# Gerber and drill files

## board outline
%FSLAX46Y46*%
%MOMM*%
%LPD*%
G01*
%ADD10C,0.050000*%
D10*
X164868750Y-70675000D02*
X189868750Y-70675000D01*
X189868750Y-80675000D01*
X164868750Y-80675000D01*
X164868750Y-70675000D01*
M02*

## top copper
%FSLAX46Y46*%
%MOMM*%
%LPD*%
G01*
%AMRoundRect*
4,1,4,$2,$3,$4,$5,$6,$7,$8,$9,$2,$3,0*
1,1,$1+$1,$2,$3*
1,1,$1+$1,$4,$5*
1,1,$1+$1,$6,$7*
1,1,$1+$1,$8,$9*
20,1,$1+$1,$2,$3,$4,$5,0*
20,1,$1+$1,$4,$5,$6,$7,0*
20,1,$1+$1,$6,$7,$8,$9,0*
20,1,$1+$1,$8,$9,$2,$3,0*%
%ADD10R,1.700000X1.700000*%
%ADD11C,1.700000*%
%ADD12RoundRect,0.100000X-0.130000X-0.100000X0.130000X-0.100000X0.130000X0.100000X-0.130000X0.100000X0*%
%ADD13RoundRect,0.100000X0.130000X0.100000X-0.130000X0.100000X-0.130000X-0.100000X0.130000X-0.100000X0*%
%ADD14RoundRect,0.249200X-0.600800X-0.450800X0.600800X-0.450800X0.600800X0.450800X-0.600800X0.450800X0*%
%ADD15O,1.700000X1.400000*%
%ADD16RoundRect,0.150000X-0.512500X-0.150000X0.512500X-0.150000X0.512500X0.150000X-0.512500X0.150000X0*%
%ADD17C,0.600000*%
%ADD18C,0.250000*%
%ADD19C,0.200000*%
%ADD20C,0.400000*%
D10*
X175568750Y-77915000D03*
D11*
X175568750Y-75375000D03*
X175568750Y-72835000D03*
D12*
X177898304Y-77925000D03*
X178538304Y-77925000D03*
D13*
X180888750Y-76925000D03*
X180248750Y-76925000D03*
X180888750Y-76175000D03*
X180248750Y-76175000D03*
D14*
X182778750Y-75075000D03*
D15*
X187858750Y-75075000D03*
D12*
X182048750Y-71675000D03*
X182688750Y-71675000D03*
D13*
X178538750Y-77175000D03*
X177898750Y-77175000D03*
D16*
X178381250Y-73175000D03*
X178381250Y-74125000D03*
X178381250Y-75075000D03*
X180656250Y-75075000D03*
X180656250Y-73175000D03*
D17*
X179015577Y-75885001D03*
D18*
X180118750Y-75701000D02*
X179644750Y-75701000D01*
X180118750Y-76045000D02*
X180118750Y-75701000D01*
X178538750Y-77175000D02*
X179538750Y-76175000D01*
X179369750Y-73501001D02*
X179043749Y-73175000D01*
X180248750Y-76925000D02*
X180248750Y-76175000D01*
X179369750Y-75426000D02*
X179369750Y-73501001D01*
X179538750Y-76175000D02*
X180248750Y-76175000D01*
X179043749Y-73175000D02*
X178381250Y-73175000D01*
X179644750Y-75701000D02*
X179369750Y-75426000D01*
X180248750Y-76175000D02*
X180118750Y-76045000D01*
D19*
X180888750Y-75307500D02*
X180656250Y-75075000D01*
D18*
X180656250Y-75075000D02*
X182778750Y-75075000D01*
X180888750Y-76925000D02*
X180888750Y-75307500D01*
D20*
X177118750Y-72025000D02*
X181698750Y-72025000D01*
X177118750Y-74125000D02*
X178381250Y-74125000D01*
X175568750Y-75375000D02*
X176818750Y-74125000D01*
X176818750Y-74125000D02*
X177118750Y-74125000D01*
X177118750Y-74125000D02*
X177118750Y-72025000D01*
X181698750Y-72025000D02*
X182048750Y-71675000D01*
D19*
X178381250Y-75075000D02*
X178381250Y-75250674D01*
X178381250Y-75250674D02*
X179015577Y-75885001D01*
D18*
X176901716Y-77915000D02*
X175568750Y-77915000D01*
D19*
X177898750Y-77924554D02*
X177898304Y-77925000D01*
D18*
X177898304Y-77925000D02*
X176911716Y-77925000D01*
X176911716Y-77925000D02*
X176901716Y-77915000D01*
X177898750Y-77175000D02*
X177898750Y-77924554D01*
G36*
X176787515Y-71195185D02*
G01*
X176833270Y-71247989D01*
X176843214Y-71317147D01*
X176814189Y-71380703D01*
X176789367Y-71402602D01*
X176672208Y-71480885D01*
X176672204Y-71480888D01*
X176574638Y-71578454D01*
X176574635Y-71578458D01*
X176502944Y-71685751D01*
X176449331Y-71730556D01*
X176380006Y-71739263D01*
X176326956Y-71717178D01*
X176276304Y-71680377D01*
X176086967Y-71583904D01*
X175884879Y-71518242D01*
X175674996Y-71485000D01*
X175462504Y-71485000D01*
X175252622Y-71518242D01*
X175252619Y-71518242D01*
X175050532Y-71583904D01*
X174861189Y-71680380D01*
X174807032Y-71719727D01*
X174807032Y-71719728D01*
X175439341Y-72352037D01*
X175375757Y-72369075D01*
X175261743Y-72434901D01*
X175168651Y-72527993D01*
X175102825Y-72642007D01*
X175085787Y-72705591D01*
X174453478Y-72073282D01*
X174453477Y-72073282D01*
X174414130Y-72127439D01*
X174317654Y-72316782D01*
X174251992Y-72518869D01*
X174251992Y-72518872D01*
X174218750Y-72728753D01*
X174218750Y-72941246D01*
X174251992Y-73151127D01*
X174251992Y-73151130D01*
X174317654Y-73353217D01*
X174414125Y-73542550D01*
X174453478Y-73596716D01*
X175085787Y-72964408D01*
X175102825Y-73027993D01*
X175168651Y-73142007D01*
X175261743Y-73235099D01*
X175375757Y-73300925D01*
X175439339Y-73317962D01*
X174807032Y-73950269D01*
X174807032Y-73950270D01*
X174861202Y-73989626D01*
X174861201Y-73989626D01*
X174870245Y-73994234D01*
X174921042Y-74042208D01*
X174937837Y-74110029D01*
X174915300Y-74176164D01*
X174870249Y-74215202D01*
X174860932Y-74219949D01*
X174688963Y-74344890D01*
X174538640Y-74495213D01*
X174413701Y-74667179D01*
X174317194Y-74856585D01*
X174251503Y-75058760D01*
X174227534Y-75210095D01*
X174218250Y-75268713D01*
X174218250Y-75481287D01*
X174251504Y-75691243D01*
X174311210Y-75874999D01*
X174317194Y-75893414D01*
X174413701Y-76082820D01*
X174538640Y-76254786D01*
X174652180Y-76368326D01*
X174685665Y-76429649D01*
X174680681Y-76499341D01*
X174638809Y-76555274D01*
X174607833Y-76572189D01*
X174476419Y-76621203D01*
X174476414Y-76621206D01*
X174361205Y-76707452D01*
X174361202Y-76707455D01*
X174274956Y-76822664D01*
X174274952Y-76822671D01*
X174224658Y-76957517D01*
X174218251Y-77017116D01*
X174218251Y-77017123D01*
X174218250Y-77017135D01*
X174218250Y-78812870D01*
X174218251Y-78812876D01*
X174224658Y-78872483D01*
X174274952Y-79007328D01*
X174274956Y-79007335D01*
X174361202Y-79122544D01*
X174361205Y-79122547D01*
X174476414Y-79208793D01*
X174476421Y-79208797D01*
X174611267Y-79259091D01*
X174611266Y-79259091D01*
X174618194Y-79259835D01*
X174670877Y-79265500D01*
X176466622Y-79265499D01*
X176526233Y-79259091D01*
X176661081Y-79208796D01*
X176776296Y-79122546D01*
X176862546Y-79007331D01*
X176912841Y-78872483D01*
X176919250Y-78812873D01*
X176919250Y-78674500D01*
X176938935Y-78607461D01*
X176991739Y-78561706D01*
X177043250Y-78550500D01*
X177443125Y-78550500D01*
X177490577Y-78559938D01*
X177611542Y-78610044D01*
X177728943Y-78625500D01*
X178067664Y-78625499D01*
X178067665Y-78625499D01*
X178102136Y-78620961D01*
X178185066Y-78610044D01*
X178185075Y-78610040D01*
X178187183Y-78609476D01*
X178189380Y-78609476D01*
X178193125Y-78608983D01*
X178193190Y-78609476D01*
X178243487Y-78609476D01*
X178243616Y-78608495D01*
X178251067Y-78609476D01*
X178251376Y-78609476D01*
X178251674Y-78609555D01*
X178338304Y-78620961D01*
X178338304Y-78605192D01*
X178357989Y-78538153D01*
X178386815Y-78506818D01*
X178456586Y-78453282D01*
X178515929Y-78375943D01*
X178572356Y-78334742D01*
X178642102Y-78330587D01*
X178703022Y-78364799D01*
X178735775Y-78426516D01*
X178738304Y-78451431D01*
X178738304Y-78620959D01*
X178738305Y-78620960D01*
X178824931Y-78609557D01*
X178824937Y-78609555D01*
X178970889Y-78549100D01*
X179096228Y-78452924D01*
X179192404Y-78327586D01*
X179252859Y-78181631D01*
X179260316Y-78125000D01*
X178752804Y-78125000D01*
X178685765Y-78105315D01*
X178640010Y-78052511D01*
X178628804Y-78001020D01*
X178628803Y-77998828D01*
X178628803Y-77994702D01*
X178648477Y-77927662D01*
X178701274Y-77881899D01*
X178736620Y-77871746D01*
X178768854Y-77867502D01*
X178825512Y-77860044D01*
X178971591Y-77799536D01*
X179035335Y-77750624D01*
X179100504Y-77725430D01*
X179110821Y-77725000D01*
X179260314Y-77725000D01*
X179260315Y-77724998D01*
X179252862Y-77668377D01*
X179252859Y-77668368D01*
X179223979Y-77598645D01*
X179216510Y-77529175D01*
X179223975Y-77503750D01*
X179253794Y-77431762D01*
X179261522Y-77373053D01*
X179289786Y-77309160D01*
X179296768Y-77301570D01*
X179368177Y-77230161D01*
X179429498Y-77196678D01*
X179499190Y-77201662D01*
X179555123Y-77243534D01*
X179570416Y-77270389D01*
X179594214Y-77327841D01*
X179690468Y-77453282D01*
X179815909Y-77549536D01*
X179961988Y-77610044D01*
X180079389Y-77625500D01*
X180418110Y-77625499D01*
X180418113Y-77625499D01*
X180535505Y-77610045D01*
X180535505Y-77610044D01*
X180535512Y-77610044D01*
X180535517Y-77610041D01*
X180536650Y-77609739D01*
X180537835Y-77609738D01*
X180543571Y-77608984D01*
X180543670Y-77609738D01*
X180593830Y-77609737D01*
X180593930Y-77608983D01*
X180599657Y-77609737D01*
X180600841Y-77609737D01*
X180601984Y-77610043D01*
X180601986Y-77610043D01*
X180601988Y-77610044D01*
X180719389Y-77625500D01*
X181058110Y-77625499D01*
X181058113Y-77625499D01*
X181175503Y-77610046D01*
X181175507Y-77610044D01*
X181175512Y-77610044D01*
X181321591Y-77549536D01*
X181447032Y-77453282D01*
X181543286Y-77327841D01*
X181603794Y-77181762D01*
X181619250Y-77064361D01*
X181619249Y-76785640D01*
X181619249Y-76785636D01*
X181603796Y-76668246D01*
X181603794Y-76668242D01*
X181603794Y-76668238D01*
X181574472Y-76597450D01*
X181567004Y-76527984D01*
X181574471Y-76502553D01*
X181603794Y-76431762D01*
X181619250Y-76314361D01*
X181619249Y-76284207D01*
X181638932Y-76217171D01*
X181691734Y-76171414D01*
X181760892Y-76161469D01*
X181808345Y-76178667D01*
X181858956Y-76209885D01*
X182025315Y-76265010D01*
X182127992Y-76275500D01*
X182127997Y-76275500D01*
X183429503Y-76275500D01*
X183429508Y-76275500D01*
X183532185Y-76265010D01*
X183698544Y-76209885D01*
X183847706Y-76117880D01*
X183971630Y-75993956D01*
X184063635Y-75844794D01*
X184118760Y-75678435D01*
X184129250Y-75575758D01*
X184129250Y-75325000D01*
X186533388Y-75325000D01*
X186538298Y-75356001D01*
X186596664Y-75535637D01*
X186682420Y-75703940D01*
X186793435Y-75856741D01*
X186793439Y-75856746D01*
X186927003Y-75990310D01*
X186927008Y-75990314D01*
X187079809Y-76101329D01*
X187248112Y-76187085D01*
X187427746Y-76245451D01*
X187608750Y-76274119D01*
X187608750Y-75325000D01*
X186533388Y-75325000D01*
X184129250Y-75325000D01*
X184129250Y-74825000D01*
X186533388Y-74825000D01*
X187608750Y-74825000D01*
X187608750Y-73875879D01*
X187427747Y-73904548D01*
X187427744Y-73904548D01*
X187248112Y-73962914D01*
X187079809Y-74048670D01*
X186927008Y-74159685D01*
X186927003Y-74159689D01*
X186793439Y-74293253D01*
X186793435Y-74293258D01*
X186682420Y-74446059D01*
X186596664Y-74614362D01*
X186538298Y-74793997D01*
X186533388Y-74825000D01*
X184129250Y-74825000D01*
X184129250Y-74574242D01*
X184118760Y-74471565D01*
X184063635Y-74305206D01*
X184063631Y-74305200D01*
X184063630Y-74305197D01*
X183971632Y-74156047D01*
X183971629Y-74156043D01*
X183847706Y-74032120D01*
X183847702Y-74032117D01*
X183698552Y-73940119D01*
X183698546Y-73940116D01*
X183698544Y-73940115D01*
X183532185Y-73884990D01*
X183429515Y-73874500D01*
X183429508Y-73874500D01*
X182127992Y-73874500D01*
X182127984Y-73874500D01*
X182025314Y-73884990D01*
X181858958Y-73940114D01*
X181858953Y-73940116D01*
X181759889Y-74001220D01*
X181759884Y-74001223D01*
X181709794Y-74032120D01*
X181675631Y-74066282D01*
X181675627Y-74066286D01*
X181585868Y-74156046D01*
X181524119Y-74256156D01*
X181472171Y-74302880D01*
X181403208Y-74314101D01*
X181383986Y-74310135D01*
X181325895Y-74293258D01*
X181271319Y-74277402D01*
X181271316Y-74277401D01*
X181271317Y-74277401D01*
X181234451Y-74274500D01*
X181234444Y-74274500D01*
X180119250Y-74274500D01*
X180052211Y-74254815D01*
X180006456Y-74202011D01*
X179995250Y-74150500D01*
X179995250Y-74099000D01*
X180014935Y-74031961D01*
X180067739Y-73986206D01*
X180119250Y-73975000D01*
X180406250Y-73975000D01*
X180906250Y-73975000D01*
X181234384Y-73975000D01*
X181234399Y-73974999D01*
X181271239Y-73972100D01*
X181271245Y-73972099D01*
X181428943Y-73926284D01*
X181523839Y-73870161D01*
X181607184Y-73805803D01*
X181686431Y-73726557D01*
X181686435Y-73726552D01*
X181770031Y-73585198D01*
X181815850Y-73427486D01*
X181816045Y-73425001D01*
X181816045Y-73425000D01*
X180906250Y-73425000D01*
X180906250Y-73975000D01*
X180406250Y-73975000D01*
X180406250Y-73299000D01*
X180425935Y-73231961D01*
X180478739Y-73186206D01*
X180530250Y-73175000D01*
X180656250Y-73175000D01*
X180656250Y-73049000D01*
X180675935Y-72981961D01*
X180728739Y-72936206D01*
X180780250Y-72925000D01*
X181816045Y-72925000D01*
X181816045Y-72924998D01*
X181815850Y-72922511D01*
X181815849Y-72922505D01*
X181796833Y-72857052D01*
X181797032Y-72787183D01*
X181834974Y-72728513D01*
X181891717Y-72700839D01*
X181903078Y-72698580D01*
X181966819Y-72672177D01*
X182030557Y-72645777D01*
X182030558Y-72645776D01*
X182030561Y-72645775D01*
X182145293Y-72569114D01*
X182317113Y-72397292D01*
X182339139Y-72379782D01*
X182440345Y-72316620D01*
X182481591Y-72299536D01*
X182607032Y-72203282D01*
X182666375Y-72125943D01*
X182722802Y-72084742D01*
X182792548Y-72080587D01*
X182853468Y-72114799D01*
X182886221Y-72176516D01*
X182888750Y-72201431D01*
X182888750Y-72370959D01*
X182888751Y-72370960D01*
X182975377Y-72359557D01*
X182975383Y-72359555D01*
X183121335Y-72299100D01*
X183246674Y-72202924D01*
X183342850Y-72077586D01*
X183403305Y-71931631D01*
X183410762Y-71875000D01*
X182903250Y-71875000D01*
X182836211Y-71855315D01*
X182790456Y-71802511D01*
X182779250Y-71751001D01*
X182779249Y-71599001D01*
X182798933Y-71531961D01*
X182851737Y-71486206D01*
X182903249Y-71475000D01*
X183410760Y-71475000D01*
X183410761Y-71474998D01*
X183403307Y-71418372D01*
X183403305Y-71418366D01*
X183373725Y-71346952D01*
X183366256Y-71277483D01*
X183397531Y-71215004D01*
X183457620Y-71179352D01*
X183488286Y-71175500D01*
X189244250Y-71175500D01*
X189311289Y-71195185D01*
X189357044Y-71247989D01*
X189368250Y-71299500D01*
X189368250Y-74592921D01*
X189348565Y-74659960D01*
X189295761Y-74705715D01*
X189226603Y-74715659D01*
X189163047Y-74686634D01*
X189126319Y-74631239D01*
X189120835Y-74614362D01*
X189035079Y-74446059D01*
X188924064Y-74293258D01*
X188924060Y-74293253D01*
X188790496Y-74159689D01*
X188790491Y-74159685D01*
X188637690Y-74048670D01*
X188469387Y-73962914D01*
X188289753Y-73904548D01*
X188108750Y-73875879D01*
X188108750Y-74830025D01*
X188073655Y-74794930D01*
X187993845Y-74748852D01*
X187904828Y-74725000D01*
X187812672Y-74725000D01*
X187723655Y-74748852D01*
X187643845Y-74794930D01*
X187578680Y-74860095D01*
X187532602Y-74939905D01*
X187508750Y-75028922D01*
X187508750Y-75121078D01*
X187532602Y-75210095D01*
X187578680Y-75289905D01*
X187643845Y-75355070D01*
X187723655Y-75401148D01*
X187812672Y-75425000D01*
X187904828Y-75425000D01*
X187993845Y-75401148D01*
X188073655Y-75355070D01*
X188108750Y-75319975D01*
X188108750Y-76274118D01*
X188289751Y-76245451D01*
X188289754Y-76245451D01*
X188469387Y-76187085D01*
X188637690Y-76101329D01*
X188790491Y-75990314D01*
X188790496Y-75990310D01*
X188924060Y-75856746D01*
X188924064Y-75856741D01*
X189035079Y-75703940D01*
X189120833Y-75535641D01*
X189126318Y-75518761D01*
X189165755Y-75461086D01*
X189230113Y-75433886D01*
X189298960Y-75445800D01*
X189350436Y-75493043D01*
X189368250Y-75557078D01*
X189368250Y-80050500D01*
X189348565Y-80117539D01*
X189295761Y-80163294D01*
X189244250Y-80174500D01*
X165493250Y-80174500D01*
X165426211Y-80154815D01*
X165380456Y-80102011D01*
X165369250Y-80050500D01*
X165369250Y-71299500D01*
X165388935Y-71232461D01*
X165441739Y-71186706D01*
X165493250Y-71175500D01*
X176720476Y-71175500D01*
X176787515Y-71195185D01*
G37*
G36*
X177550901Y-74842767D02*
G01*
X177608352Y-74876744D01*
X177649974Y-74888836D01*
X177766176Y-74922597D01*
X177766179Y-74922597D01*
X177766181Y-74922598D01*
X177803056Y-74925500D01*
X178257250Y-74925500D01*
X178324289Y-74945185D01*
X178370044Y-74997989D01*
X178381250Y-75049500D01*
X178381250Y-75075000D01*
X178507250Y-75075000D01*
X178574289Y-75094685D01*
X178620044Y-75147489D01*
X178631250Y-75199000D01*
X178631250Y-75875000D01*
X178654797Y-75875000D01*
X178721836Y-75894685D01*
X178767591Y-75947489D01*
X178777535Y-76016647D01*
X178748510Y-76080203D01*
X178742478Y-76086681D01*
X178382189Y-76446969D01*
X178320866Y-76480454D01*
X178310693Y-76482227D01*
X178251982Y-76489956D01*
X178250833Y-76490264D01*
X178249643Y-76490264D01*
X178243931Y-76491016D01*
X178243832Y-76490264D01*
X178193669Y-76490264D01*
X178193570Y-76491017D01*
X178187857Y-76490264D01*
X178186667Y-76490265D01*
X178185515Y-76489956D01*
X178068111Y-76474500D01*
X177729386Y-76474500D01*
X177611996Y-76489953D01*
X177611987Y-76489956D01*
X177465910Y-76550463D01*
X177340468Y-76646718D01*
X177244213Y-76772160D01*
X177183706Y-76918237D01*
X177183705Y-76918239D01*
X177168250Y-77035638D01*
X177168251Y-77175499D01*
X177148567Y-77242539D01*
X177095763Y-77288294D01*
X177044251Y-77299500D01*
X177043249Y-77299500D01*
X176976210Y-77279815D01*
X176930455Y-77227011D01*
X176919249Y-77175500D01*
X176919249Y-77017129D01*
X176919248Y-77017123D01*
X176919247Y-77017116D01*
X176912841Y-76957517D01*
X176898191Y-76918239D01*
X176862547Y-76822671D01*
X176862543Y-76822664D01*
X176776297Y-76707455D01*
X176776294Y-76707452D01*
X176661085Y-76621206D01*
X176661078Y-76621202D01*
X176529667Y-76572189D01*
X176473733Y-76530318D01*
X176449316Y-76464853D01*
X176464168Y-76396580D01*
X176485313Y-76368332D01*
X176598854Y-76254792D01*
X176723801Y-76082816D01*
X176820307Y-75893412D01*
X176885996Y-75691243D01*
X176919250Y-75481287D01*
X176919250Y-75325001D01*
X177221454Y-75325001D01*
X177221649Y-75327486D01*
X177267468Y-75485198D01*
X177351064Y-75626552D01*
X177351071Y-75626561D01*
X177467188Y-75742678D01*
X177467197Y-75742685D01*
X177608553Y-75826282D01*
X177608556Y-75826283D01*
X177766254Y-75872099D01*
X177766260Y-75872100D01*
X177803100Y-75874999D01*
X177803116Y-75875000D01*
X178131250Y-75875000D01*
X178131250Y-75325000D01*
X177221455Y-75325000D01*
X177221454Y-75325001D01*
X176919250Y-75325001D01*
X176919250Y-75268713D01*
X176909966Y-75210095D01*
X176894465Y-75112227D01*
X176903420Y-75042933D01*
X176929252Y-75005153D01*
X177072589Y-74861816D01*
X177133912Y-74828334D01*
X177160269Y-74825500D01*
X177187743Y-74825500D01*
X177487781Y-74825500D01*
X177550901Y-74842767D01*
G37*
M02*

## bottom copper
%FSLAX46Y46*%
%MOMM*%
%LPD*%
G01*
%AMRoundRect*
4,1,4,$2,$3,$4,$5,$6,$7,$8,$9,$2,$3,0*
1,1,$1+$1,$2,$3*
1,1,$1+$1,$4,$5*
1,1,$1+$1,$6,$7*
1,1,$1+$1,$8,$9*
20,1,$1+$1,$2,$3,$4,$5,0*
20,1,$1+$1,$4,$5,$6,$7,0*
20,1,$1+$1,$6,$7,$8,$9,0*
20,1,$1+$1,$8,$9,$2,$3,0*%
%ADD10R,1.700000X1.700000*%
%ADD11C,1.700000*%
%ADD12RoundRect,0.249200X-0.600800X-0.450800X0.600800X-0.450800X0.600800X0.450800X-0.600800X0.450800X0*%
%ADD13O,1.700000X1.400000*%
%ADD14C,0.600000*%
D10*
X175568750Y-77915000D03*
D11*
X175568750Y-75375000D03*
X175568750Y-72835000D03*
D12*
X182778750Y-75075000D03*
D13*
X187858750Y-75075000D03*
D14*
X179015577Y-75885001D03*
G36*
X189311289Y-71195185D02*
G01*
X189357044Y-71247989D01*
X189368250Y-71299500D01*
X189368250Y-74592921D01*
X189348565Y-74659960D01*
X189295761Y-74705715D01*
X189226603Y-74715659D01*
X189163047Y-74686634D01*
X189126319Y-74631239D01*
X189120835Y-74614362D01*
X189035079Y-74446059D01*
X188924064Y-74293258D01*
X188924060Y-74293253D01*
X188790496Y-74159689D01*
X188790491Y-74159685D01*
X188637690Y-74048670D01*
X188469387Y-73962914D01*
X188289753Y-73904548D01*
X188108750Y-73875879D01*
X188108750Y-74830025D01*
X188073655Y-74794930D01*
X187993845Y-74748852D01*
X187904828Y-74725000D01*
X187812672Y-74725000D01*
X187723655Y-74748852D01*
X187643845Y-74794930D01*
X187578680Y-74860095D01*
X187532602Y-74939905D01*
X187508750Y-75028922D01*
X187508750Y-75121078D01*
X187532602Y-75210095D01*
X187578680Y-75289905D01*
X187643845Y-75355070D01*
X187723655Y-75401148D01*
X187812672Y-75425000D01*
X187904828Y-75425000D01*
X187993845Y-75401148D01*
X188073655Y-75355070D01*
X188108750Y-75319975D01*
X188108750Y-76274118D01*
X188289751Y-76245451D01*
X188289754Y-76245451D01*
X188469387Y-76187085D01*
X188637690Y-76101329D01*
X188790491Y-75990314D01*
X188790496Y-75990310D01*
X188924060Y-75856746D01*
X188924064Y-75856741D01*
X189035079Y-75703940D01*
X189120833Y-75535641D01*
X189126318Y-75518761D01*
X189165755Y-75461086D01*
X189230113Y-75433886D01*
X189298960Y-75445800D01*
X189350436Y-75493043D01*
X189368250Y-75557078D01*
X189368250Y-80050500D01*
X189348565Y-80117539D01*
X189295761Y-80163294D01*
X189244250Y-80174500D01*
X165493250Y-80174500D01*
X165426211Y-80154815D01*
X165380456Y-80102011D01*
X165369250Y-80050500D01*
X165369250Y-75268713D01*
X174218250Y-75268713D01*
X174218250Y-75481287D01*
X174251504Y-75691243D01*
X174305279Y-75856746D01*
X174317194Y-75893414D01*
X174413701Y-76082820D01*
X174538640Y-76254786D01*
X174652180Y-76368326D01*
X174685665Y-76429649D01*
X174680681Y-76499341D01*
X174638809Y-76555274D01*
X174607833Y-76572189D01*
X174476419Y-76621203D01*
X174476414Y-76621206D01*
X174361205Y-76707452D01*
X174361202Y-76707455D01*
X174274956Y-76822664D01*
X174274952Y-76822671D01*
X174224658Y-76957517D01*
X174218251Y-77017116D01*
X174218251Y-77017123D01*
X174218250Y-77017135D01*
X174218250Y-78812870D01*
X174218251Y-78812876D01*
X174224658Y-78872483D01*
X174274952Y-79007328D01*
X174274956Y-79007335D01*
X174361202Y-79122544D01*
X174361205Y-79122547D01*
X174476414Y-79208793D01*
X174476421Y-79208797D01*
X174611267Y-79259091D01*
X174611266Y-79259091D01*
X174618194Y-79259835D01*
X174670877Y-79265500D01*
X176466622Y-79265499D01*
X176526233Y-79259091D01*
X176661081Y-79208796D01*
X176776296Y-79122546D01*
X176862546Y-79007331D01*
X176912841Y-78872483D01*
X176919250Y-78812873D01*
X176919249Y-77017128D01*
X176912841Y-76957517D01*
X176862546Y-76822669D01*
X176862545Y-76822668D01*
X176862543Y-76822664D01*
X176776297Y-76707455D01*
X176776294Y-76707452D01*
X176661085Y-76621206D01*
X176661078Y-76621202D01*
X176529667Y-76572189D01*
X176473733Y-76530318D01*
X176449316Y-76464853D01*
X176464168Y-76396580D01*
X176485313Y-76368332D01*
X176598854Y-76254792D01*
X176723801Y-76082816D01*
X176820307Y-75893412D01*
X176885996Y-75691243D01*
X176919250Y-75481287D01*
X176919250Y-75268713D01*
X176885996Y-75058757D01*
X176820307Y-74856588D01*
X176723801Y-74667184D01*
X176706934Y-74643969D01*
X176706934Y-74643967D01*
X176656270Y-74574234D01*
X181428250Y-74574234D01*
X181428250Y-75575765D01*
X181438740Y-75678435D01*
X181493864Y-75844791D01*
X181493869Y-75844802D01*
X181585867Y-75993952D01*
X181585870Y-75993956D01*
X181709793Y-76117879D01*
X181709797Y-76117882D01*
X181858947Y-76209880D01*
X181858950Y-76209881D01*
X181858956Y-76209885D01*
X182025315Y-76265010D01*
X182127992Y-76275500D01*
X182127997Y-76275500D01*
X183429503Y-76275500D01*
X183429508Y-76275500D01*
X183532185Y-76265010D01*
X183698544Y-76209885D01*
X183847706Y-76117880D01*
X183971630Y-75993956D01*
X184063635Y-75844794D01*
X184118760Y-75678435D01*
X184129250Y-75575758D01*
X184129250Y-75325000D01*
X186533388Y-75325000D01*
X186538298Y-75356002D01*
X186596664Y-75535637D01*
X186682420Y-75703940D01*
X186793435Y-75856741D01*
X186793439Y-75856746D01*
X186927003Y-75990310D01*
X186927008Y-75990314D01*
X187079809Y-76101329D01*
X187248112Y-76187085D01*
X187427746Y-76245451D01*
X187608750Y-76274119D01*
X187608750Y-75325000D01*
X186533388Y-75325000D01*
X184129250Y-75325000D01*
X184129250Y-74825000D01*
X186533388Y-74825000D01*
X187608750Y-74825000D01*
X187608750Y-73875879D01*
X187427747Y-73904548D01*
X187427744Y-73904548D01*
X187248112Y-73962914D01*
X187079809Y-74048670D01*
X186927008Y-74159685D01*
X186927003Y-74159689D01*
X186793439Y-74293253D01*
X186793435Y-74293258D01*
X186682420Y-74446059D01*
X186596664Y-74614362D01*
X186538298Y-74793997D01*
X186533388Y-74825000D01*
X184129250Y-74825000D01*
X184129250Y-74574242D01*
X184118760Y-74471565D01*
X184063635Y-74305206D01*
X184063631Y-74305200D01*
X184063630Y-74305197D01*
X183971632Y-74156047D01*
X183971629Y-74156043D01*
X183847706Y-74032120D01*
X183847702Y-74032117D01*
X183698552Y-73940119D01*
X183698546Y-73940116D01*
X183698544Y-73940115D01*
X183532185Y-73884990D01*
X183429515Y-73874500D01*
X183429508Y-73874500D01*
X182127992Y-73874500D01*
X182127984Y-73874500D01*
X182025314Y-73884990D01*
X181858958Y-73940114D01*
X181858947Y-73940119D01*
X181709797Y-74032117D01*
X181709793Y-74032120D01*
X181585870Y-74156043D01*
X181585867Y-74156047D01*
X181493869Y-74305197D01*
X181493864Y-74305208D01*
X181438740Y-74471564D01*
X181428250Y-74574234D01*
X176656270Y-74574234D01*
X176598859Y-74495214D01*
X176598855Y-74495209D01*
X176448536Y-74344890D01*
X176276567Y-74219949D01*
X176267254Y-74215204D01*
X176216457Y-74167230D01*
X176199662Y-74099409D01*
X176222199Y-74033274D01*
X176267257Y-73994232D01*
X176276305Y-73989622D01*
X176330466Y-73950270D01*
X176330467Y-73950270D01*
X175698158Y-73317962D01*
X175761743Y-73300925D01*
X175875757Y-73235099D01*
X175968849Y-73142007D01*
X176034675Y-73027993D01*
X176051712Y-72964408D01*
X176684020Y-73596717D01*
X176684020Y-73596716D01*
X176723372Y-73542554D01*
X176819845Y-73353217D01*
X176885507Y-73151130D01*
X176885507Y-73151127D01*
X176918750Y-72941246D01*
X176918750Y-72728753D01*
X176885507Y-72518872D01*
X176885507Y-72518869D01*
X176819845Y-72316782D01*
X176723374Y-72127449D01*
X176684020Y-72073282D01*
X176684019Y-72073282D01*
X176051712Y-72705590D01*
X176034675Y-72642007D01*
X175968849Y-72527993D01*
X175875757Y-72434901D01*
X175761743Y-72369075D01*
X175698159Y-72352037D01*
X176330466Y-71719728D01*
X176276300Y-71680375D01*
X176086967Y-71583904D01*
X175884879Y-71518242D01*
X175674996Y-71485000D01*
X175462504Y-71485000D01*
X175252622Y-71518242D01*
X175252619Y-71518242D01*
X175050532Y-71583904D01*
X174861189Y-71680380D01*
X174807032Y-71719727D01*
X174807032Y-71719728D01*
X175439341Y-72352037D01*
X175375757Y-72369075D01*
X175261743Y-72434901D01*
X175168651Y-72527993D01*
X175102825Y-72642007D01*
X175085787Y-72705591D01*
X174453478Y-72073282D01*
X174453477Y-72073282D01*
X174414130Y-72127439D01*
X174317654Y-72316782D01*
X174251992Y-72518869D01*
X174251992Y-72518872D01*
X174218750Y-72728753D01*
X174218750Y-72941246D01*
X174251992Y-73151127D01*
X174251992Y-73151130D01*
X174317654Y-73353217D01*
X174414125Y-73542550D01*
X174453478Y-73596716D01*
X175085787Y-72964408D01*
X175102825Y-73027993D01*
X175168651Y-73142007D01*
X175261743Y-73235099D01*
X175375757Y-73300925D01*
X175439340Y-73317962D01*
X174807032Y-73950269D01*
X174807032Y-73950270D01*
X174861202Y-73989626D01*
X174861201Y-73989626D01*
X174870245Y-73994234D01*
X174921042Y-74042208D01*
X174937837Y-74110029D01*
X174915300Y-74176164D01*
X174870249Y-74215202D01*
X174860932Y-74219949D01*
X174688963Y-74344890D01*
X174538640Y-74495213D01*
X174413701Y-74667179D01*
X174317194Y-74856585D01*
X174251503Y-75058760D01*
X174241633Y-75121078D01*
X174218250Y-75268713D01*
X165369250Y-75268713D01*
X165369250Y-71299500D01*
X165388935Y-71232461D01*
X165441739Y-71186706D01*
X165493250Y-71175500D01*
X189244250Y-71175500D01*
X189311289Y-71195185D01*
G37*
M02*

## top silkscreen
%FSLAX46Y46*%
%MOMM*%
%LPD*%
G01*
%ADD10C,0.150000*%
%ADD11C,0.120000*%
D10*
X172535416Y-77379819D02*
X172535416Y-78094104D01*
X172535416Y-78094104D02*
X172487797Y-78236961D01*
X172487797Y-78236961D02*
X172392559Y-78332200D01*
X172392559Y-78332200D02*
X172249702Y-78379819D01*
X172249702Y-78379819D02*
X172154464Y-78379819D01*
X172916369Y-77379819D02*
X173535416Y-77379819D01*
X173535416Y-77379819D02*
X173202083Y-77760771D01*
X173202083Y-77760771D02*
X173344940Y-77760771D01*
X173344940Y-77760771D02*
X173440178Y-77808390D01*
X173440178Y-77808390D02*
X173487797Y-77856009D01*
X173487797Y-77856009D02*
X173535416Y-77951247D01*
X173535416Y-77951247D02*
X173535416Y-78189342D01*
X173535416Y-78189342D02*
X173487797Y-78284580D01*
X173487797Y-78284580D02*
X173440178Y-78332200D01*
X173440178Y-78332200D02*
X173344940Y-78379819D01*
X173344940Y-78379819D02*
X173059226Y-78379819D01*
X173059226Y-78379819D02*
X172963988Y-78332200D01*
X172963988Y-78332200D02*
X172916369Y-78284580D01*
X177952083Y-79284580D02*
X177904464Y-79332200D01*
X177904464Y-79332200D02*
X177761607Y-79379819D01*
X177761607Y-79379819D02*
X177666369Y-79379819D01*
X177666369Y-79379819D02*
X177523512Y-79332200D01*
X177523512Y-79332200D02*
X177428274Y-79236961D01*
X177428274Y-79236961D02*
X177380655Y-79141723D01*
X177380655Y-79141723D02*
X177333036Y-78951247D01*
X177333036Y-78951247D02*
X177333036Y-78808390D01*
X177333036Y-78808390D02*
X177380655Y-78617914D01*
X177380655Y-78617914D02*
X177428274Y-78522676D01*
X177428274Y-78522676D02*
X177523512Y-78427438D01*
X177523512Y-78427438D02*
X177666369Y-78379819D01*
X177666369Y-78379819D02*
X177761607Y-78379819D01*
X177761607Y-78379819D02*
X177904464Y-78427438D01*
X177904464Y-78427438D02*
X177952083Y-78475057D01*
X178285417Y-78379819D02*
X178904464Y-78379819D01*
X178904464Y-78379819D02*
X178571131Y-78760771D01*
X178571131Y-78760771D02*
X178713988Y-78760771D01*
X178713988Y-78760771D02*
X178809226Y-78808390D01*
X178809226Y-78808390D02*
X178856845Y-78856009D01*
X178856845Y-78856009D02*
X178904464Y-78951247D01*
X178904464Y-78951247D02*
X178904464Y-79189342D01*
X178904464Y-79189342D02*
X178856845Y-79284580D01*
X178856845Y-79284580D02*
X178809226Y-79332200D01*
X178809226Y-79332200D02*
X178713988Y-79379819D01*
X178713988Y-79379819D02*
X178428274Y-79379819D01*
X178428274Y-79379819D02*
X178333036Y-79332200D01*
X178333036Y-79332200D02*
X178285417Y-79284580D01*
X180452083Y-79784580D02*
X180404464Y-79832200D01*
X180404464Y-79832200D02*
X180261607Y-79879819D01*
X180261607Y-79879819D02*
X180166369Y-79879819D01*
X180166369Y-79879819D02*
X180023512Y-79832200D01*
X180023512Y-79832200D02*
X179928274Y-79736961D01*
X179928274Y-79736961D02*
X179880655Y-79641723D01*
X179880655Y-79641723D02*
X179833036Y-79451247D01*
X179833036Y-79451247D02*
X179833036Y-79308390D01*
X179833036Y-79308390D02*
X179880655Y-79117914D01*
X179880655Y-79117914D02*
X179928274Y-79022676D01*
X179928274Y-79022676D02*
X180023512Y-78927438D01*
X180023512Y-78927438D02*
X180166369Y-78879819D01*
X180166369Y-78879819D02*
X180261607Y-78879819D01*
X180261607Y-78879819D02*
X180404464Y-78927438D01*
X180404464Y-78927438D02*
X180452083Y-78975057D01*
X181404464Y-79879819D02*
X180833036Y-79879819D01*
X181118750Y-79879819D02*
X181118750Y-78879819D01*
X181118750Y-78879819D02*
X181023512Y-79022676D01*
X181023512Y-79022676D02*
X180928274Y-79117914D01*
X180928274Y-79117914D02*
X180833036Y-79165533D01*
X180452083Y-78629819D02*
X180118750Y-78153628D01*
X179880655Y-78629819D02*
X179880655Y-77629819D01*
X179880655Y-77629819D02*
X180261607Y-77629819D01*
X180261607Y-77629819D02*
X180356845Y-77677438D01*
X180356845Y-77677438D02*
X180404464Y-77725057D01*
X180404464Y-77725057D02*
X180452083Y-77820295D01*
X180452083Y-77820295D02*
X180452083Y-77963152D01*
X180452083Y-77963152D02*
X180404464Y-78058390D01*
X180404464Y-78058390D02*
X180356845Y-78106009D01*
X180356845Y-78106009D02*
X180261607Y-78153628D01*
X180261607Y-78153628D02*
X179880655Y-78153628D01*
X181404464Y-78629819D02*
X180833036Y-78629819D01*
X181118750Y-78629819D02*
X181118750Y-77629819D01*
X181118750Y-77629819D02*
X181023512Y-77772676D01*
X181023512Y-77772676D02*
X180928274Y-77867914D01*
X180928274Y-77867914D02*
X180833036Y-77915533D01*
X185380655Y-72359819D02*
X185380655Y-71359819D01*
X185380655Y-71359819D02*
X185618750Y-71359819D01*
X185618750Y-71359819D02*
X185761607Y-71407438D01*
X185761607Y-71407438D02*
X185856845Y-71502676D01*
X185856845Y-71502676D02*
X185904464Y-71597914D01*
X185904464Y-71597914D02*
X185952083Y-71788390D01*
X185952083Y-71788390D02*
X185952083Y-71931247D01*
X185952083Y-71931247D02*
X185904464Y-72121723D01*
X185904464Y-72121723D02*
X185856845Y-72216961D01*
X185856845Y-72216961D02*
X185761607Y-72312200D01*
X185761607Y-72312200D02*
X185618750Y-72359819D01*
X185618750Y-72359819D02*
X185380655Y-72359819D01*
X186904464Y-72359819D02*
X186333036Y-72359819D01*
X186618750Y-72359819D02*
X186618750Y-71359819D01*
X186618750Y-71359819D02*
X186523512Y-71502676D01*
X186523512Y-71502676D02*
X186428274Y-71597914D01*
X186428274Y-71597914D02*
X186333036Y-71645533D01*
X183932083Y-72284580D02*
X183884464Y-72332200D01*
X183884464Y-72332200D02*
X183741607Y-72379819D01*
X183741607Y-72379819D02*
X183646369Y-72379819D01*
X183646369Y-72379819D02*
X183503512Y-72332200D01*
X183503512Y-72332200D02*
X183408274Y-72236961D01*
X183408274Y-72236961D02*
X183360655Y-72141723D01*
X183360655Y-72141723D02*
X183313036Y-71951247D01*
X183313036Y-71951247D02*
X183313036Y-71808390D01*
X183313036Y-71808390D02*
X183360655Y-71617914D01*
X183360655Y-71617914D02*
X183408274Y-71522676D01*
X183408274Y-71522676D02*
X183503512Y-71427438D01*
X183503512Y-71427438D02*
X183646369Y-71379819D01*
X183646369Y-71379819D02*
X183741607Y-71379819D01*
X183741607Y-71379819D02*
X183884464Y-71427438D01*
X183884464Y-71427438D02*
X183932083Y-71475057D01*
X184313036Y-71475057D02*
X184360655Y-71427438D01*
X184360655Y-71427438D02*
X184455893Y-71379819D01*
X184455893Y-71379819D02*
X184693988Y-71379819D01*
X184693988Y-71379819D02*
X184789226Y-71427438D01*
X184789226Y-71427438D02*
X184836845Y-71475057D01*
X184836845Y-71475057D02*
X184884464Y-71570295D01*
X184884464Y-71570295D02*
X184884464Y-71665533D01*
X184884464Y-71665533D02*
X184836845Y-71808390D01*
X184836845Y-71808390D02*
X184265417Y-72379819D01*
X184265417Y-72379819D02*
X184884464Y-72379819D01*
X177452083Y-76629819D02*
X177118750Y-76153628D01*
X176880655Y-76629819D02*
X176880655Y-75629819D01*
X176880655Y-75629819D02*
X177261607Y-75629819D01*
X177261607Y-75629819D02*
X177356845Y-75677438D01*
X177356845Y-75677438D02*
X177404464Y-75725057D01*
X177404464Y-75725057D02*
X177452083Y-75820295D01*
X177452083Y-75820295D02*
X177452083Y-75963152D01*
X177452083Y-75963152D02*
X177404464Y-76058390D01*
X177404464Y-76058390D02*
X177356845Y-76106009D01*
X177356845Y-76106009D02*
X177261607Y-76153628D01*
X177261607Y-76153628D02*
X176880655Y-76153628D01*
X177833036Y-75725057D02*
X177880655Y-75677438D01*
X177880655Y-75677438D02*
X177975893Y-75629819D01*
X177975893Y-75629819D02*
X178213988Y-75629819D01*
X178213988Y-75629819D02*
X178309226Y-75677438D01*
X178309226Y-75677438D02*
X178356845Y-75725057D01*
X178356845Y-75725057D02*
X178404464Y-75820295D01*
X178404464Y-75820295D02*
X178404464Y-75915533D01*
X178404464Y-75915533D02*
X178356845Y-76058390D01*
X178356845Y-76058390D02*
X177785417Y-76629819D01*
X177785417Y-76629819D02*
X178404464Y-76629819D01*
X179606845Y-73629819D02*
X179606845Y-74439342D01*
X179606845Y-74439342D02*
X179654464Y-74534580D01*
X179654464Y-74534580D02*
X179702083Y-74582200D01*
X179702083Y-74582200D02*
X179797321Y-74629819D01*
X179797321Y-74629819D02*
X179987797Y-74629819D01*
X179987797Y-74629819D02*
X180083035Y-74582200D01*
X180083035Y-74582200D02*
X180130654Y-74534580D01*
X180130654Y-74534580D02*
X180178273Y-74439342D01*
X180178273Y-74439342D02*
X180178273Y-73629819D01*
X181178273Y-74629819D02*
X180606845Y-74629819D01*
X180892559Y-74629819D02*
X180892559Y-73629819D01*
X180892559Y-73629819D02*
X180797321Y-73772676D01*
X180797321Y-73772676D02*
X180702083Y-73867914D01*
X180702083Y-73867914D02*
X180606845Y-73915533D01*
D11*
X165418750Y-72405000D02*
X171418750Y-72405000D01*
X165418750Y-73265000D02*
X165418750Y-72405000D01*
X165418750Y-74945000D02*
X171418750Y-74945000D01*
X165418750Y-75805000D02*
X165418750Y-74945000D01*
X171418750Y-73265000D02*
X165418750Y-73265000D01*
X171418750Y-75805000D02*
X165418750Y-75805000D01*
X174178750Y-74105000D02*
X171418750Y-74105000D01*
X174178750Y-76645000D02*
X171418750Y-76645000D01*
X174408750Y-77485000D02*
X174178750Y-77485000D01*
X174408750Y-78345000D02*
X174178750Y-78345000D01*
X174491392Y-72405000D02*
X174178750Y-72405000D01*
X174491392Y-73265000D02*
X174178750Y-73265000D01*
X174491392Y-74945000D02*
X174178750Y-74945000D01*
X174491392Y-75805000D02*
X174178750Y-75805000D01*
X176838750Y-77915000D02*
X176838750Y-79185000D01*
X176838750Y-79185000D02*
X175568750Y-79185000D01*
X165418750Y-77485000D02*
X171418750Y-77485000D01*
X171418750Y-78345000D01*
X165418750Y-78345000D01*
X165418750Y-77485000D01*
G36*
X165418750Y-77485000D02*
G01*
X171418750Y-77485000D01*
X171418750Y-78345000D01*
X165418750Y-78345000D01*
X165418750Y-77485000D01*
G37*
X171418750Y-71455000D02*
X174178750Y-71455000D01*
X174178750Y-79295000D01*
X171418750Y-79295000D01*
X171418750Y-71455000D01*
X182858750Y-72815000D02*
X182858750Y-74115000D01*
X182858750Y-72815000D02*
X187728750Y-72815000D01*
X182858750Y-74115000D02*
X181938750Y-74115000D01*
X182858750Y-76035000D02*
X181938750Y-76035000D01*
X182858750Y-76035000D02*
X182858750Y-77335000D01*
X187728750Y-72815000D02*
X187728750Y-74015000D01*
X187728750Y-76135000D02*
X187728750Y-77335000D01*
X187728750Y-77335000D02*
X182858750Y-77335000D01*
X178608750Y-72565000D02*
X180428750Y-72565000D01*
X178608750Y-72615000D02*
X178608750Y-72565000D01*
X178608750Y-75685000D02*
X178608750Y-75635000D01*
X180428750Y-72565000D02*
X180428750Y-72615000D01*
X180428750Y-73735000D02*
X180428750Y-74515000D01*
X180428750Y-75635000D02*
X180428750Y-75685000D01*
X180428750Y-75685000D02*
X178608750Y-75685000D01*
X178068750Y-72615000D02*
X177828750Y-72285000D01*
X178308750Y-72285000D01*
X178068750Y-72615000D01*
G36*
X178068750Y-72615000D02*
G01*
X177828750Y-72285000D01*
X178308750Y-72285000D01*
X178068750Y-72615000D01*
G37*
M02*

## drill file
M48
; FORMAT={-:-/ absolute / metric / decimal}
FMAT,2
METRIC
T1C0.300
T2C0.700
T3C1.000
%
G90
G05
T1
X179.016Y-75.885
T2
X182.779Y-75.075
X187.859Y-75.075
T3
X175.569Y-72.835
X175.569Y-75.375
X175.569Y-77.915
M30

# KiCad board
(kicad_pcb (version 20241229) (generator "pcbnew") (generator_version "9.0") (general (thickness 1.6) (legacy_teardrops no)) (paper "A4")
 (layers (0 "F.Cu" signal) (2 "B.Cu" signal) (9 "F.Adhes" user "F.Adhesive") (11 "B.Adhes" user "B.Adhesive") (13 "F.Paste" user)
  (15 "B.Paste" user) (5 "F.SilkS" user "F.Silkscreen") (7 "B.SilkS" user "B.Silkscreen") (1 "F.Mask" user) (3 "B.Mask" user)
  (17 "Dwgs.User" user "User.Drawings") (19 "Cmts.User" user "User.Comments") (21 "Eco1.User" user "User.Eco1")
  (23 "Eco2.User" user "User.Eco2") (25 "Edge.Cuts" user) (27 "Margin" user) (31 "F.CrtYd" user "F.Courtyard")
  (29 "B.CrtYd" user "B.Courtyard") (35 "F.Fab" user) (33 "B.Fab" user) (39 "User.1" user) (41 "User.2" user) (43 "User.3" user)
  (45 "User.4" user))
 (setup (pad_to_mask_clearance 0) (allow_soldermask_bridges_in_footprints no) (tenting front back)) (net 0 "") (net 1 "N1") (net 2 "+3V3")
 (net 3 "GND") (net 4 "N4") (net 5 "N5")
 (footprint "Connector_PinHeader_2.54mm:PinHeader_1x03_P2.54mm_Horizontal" (layer "F.Cu") (at 175.56875 77.915 180)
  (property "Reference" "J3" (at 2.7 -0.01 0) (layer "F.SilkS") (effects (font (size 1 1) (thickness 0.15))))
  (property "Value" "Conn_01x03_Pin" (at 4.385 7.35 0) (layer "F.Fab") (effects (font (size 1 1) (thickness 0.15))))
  (fp_line (start 10.15 5.51) (end 4.15 5.51) (stroke (width 0.12) (type solid)) (layer "F.SilkS"))
  (fp_line (start 10.15 4.65) (end 10.15 5.51) (stroke (width 0.12) (type solid)) (layer "F.SilkS"))
  (fp_line (start 10.15 2.97) (end 4.15 2.97) (stroke (width 0.12) (type solid)) (layer "F.SilkS"))
  (fp_line (start 10.15 2.11) (end 10.15 2.97) (stroke (width 0.12) (type solid)) (layer "F.SilkS"))
  (fp_line (start 4.15 4.65) (end 10.15 4.65) (stroke (width 0.12) (type solid)) (layer "F.SilkS"))
  (fp_line (start 4.15 2.11) (end 10.15 2.11) (stroke (width 0.12) (type solid)) (layer "F.SilkS"))
  (fp_line (start 1.39 3.81) (end 4.15 3.81) (stroke (width 0.12) (type solid)) (layer "F.SilkS"))
  (fp_line (start 1.39 1.27) (end 4.15 1.27) (stroke (width 0.12) (type solid)) (layer "F.SilkS"))
  (fp_line (start 1.16 0.43) (end 1.39 0.43) (stroke (width 0.12) (type solid)) (layer "F.SilkS"))
  (fp_line (start 1.16 -0.43) (end 1.39 -0.43) (stroke (width 0.12) (type solid)) (layer "F.SilkS"))
  (fp_line (start 1.077358 5.51) (end 1.39 5.51) (stroke (width 0.12) (type solid)) (layer "F.SilkS"))
  (fp_line (start 1.077358 4.65) (end 1.39 4.65) (stroke (width 0.12) (type solid)) (layer "F.SilkS"))
  (fp_line (start 1.077358 2.97) (end 1.39 2.97) (stroke (width 0.12) (type solid)) (layer "F.SilkS"))
  (fp_line (start 1.077358 2.11) (end 1.39 2.11) (stroke (width 0.12) (type solid)) (layer "F.SilkS"))
  (fp_line (start -1.27 0) (end -1.27 -1.27) (stroke (width 0.12) (type solid)) (layer "F.SilkS"))
  (fp_line (start -1.27 -1.27) (end 0 -1.27) (stroke (width 0.12) (type solid)) (layer "F.SilkS"))
  (fp_rect (start 4.15 -0.43) (end 10.15 0.43) (stroke (width 0.12) (type solid)) (fill yes) (layer "F.SilkS"))
  (fp_rect (start 1.39 -1.38) (end 4.15 6.46) (stroke (width 0.12) (type solid)) (fill no) (layer "F.SilkS"))
  (pad "1" thru_hole rect (at 0 0 180) (size 1.7 1.7) (drill 1) (layers "*.Cu" "*.Mask") (remove_unused_layers no) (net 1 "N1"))
  (pad "2" thru_hole circle (at 0 2.54 180) (size 1.7 1.7) (drill 1) (layers "*.Cu" "*.Mask") (remove_unused_layers no) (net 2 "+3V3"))
  (pad "3" thru_hole circle (at 0 5.08 180) (size 1.7 1.7) (drill 1) (layers "*.Cu" "*.Mask") (remove_unused_layers no) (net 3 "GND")))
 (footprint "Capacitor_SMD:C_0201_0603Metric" (layer "F.Cu") (at 178.218304 77.925)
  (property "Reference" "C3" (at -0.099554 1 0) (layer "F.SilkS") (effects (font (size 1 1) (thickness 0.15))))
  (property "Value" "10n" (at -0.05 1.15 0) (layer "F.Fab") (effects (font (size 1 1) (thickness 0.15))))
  (pad "" smd roundrect (at -0.345 0) (size 0.318 0.36) (layers "F.Paste") (roundrect_rratio 0.25))
  (pad "" smd roundrect (at 0.345 0) (size 0.318 0.36) (layers "F.Paste") (roundrect_rratio 0.25))
  (pad "1" smd roundrect (at -0.32 0) (size 0.46 0.4) (layers "F.Cu" "F.Mask") (roundrect_rratio 0.25) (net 1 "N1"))
  (pad "2" smd roundrect (at 0.32 0) (size 0.46 0.4) (layers "F.Cu" "F.Mask") (roundrect_rratio 0.25) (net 3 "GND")))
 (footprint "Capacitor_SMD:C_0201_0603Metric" (layer "F.Cu") (at 180.56875 76.925 180)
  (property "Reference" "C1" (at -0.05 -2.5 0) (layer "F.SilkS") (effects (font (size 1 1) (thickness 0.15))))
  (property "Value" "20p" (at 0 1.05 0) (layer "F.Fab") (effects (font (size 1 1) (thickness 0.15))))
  (pad "" smd roundrect (at -0.345 0 180) (size 0.318 0.36) (layers "F.Paste") (roundrect_rratio 0.25))
  (pad "" smd roundrect (at 0.345 0 180) (size 0.318 0.36) (layers "F.Paste") (roundrect_rratio 0.25))
  (pad "1" smd roundrect (at -0.32 0 180) (size 0.46 0.4) (layers "F.Cu" "F.Mask") (roundrect_rratio 0.25) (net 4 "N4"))
  (pad "2" smd roundrect (at 0.32 0 180) (size 0.46 0.4) (layers "F.Cu" "F.Mask") (roundrect_rratio 0.25) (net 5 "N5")))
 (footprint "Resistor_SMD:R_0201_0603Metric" (layer "F.Cu") (at 180.56875 76.175 180)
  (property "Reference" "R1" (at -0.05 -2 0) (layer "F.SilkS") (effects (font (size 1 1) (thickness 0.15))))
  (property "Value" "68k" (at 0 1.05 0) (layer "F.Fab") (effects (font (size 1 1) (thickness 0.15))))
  (pad "" smd roundrect (at -0.345 0 180) (size 0.318 0.36) (layers "F.Paste") (roundrect_rratio 0.25))
  (pad "" smd roundrect (at 0.345 0 180) (size 0.318 0.36) (layers "F.Paste") (roundrect_rratio 0.25))
  (pad "1" smd roundrect (at -0.32 0 180) (size 0.46 0.4) (layers "F.Cu" "F.Mask") (roundrect_rratio 0.25) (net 4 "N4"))
  (pad "2" smd roundrect (at 0.32 0 180) (size 0.46 0.4) (layers "F.Cu" "F.Mask") (roundrect_rratio 0.25) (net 5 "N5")))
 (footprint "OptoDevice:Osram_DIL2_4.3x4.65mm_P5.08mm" (layer "F.Cu") (at 182.77875 75.075)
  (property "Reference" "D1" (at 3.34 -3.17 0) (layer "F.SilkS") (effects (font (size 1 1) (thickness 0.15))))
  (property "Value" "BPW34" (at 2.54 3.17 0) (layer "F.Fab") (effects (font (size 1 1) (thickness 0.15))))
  (fp_line (start 0.08 -2.26) (end 0.08 -0.96) (stroke (width 0.12) (type solid)) (layer "F.SilkS"))
  (fp_line (start 0.08 -2.26) (end 4.95 -2.26) (stroke (width 0.12) (type solid)) (layer "F.SilkS"))
  (fp_line (start 0.08 -0.96) (end -0.84 -0.96) (stroke (width 0.12) (type solid)) (layer "F.SilkS"))
  (fp_line (start 0.08 0.96) (end -0.84 0.96) (stroke (width 0.12) (type solid)) (layer "F.SilkS"))
  (fp_line (start 0.08 0.96) (end 0.08 2.26) (stroke (width 0.12) (type solid)) (layer "F.SilkS"))
  (fp_line (start 4.95 -2.26) (end 4.95 -1.06) (stroke (width 0.12) (type solid)) (layer "F.SilkS"))
  (fp_line (start 4.95 1.06) (end 4.95 2.26) (stroke (width 0.12) (type solid)) (layer "F.SilkS"))
  (fp_line (start 4.95 2.26) (end 0.08 2.26) (stroke (width 0.12) (type solid)) (layer "F.SilkS"))
  (pad "1" thru_hole roundrect (at 0 0) (size 1.7 1.4) (drill 0.7) (layers "*.Cu" "*.Mask") (remove_unused_layers no)
   (roundrect_rratio 0.178) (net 4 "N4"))
  (pad "2" thru_hole oval (at 5.08 0) (size 1.7 1.4) (drill 0.7) (layers "*.Cu" "*.Mask") (remove_unused_layers no) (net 3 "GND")))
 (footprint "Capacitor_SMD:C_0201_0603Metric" (layer "F.Cu") (at 182.36875 71.675)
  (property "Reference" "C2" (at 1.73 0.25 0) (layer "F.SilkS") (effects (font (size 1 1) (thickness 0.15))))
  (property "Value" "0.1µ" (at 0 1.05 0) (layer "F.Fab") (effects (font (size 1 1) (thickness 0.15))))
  (pad "" smd roundrect (at -0.345 0) (size 0.318 0.36) (layers "F.Paste") (roundrect_rratio 0.25))
  (pad "" smd roundrect (at 0.345 0) (size 0.318 0.36) (layers "F.Paste") (roundrect_rratio 0.25))
  (pad "1" smd roundrect (at -0.32 0) (size 0.46 0.4) (layers "F.Cu" "F.Mask") (roundrect_rratio 0.25) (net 2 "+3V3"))
  (pad "2" smd roundrect (at 0.32 0) (size 0.46 0.4) (layers "F.Cu" "F.Mask") (roundrect_rratio 0.25) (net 3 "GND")))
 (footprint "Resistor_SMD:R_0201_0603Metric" (layer "F.Cu") (at 178.21875 77.175 180)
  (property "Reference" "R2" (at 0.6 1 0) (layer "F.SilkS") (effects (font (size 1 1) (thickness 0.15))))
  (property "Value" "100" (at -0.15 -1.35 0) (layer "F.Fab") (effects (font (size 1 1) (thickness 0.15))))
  (pad "" smd roundrect (at -0.345 0 180) (size 0.318 0.36) (layers "F.Paste") (roundrect_rratio 0.25))
  (pad "" smd roundrect (at 0.345 0 180) (size 0.318 0.36) (layers "F.Paste") (roundrect_rratio 0.25))
  (pad "1" smd roundrect (at -0.32 0 180) (size 0.46 0.4) (layers "F.Cu" "F.Mask") (roundrect_rratio 0.25) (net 5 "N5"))
  (pad "2" smd roundrect (at 0.32 0 180) (size 0.46 0.4) (layers "F.Cu" "F.Mask") (roundrect_rratio 0.25) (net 1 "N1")))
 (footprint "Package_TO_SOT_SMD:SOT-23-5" (layer "F.Cu") (at 179.51875 74.125)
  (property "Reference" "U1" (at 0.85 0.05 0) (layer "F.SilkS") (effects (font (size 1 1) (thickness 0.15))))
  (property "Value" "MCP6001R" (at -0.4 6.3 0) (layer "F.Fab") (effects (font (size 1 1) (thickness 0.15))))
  (fp_line (start -0.91 -1.56) (end 0.91 -1.56) (stroke (width 0.12) (type solid)) (layer "F.SilkS"))
  (fp_line (start -0.91 -1.51) (end -0.91 -1.56) (stroke (width 0.12) (type solid)) (layer "F.SilkS"))
  (fp_line (start -0.91 1.56) (end -0.91 1.51) (stroke (width 0.12) (type solid)) (layer "F.SilkS"))
  (fp_line (start 0.91 -1.56) (end 0.91 -1.51) (stroke (width 0.12) (type solid)) (layer "F.SilkS"))
  (fp_line (start 0.91 -0.39) (end 0.91 0.39) (stroke (width 0.12) (type solid)) (layer "F.SilkS"))
  (fp_line (start 0.91 1.51) (end 0.91 1.56) (stroke (width 0.12) (type solid)) (layer "F.SilkS"))
  (fp_line (start 0.91 1.56) (end -0.91 1.56) (stroke (width 0.12) (type solid)) (layer "F.SilkS"))
  (fp_poly (pts (xy -1.45 -1.51) (xy -1.69 -1.84) (xy -1.21 -1.84)) (stroke (width 0.12) (type solid)) (fill yes) (layer "F.SilkS"))
  (pad "1" smd roundrect (at -1.1375 -0.95) (size 1.325 0.6) (layers "F.Cu" "F.Mask" "F.Paste") (roundrect_rratio 0.25) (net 5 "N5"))
  (pad "2" smd roundrect (at -1.1375 0) (size 1.325 0.6) (layers "F.Cu" "F.Mask" "F.Paste") (roundrect_rratio 0.25) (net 2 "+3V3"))
  (pad "3" smd roundrect (at -1.1375 0.95) (size 1.325 0.6) (layers "F.Cu" "F.Mask" "F.Paste") (roundrect_rratio 0.25) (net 3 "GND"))
  (pad "4" smd roundrect (at 1.1375 0.95) (size 1.325 0.6) (layers "F.Cu" "F.Mask" "F.Paste") (roundrect_rratio 0.25) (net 4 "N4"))
  (pad "5" smd roundrect (at 1.1375 -0.95) (size 1.325 0.6) (layers "F.Cu" "F.Mask" "F.Paste") (roundrect_rratio 0.25) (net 3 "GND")))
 (gr_rect (start 164.86875 70.675) (end 189.86875 80.675) (stroke (width 0.05) (type default)) (fill no) (layer "Edge.Cuts"))
 (segment (start 180.11875 75.701) (end 179.64475 75.701) (width 0.25) (layer "F.Cu") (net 5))
 (segment (start 180.11875 76.045) (end 180.11875 75.701) (width 0.25) (layer "F.Cu") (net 5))
 (segment (start 178.53875 77.175) (end 179.53875 76.175) (width 0.25) (layer "F.Cu") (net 5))
 (segment (start 179.36975 73.501001) (end 179.043749 73.175) (width 0.25) (layer "F.Cu") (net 5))
 (segment (start 180.24875 76.925) (end 180.24875 76.175) (width 0.25) (layer "F.Cu") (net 5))
 (segment (start 179.36975 75.426) (end 179.36975 73.501001) (width 0.25) (layer "F.Cu") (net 5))
 (segment (start 179.53875 76.175) (end 180.24875 76.175) (width 0.25) (layer "F.Cu") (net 5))
 (segment (start 179.043749 73.175) (end 178.38125 73.175) (width 0.25) (layer "F.Cu") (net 5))
 (segment (start 179.64475 75.701) (end 179.36975 75.426) (width 0.25) (layer "F.Cu") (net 5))
 (segment (start 180.24875 76.175) (end 180.11875 76.045) (width 0.25) (layer "F.Cu") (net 5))
 (segment (start 180.88875 75.3075) (end 180.65625 75.075) (width 0.2) (layer "F.Cu") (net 4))
 (segment (start 180.65625 75.075) (end 182.77875 75.075) (width 0.25) (layer "F.Cu") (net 4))
 (segment (start 180.88875 76.925) (end 180.88875 75.3075) (width 0.25) (layer "F.Cu") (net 4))
 (segment (start 177.11875 72.025) (end 181.69875 72.025) (width 0.4) (layer "F.Cu") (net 2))
 (segment (start 177.11875 74.125) (end 178.38125 74.125) (width 0.4) (layer "F.Cu") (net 2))
 (segment (start 175.56875 75.375) (end 176.81875 74.125) (width 0.4) (layer "F.Cu") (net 2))
 (segment (start 176.81875 74.125) (end 177.11875 74.125) (width 0.4) (layer "F.Cu") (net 2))
 (segment (start 177.11875 74.125) (end 177.11875 72.025) (width 0.4) (layer "F.Cu") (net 2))
 (segment (start 181.69875 72.025) (end 182.04875 71.675) (width 0.4) (layer "F.Cu") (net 2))
 (segment (start 178.38125 75.075) (end 178.38125 75.250674) (width 0.2) (layer "F.Cu") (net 3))
 (segment (start 178.38125 75.250674) (end 179.015577 75.885001) (width 0.2) (layer "F.Cu") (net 3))
 (via (at 179.015577 75.885001) (size 0.6) (drill 0.3) (layers "F.Cu" "B.Cu") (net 3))
 (segment (start 176.901716 77.915) (end 175.56875 77.915) (width 0.25) (layer "F.Cu") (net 1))
 (segment (start 177.89875 77.924554) (end 177.898304 77.925) (width 0.2) (layer "F.Cu") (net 1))
 (segment (start 177.898304 77.925) (end 176.911716 77.925) (width 0.25) (layer "F.Cu") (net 1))
 (segment (start 176.911716 77.925) (end 176.901716 77.915) (width 0.25) (layer "F.Cu") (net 1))
 (segment (start 177.89875 77.175) (end 177.89875 77.924554) (width 0.25) (layer "F.Cu") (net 1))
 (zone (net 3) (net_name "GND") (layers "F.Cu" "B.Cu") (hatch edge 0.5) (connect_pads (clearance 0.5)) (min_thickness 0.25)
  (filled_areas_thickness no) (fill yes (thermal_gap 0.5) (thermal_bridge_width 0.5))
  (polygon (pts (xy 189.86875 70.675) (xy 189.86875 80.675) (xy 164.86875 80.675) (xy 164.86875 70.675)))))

